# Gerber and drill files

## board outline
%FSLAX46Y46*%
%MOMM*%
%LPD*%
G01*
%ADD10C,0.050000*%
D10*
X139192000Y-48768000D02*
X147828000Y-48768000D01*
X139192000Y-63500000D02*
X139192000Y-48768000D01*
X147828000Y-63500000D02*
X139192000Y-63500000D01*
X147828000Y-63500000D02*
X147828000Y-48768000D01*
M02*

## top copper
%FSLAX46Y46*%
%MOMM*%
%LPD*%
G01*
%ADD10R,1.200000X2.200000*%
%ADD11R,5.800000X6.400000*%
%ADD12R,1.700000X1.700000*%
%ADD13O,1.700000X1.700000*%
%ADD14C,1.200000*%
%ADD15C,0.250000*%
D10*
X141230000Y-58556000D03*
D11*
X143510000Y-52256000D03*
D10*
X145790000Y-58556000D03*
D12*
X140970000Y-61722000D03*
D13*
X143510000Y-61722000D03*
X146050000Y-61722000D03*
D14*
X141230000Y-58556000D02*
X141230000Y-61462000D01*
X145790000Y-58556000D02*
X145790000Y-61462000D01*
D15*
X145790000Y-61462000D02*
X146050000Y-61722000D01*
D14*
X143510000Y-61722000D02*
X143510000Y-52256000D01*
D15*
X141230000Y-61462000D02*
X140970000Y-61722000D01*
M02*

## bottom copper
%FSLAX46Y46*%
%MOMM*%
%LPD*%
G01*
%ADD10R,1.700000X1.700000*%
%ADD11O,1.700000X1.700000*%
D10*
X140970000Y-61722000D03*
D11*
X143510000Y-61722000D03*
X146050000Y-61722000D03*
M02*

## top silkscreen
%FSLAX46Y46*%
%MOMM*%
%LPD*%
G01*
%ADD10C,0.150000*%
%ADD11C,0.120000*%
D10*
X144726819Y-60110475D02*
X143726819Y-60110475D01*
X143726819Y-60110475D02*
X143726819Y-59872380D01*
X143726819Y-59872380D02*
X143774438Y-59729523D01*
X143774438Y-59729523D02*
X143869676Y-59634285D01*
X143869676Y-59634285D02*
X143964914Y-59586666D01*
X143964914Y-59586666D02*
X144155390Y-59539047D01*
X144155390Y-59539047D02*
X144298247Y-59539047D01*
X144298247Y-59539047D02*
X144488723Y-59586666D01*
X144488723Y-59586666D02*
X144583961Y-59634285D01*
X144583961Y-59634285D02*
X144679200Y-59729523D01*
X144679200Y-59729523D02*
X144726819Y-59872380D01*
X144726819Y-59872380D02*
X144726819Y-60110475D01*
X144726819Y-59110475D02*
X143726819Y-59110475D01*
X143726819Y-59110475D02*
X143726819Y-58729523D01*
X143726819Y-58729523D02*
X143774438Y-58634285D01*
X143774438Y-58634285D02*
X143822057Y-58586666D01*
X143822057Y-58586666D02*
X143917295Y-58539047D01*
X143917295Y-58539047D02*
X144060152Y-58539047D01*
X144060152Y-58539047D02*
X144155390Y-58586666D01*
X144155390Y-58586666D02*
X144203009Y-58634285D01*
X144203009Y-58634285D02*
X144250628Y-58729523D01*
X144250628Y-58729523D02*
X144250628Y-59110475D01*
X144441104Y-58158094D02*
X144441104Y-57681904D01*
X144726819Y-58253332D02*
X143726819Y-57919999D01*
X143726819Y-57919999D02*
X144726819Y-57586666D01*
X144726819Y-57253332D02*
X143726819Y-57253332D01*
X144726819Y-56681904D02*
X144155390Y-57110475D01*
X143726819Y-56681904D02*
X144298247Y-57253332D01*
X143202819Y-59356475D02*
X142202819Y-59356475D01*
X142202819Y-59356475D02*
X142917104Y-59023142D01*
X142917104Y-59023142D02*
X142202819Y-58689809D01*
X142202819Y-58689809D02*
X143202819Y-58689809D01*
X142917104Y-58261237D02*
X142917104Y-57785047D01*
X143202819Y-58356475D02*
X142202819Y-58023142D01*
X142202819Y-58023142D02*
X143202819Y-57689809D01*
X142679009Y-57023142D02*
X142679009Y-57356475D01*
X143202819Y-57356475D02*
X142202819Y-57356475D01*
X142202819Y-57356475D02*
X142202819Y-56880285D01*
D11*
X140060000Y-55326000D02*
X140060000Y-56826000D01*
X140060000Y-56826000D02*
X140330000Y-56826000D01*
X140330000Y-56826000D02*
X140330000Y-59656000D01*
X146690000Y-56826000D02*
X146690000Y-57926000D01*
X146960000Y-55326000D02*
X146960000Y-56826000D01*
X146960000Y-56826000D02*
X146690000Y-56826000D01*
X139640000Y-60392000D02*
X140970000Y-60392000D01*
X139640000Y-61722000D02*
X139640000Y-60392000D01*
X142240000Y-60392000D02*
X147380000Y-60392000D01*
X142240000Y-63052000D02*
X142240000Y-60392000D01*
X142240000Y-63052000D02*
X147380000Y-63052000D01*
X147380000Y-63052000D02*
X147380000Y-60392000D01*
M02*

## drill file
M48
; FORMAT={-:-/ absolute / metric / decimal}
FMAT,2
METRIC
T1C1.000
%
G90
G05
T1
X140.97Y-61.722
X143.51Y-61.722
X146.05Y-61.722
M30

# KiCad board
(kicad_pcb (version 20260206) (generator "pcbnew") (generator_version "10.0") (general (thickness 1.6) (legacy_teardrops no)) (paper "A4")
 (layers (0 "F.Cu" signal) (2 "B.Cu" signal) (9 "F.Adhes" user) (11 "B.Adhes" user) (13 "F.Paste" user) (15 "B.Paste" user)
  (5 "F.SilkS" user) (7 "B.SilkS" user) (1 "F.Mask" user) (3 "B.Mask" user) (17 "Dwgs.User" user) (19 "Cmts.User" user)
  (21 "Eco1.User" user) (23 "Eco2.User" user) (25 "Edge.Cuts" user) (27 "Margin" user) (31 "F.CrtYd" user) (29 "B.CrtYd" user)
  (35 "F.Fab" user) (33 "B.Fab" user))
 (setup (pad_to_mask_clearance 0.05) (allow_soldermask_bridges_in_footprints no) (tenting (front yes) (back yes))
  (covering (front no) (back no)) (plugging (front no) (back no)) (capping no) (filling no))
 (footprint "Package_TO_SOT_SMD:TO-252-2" (layer "F.Cu") (at 143.51 54.356 90)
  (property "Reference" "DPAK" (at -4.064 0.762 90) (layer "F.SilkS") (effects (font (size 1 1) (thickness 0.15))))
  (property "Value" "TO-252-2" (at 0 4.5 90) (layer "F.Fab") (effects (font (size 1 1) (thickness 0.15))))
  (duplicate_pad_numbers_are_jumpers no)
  (fp_line (start -0.97 -3.45) (end -2.47 -3.45) (stroke (width 0.12) (type solid)) (layer "F.SilkS"))
  (fp_line (start -2.47 -3.45) (end -2.47 -3.18) (stroke (width 0.12) (type solid)) (layer "F.SilkS"))
  (fp_line (start -2.47 -3.18) (end -5.3 -3.18) (stroke (width 0.12) (type solid)) (layer "F.SilkS"))
  (fp_line (start -2.47 3.18) (end -3.57 3.18) (stroke (width 0.12) (type solid)) (layer "F.SilkS"))
  (fp_line (start -0.97 3.45) (end -2.47 3.45) (stroke (width 0.12) (type solid)) (layer "F.SilkS"))
  (fp_line (start -2.47 3.45) (end -2.47 3.18) (stroke (width 0.12) (type solid)) (layer "F.SilkS"))
  (pad "" smd rect (at 0.425 -1.525 90) (size 3.05 2.75) (layers "F.Paste"))
  (pad "" smd rect (at 0.425 1.525 90) (size 3.05 2.75) (layers "F.Paste"))
  (pad "" smd rect (at 3.775 -1.525 90) (size 3.05 2.75) (layers "F.Paste"))
  (pad "" smd rect (at 3.775 1.525 90) (size 3.05 2.75) (layers "F.Paste"))
  (pad "1" smd rect (at -4.2 -2.28 90) (size 2.2 1.2) (layers "F.Cu" "F.Mask" "F.Paste"))
  (pad "2" smd rect (at 2.1 0 90) (size 6.4 5.8) (layers "F.Cu" "F.Mask"))
  (pad "3" smd rect (at -4.2 2.28 90) (size 2.2 1.2) (layers "F.Cu" "F.Mask" "F.Paste")))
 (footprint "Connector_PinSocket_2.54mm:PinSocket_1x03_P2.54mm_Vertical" (layer "F.Cu") (at 140.97 61.722 90)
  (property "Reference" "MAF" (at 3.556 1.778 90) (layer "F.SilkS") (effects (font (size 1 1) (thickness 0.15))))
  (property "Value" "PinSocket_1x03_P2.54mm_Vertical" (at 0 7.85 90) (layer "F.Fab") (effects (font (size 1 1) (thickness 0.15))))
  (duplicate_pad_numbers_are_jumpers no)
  (fp_line (start 1.33 -1.33) (end 1.33 0) (stroke (width 0.12) (type solid)) (layer "F.SilkS"))
  (fp_line (start 0 -1.33) (end 1.33 -1.33) (stroke (width 0.12) (type solid)) (layer "F.SilkS"))
  (fp_line (start 1.33 1.27) (end 1.33 6.41) (stroke (width 0.12) (type solid)) (layer "F.SilkS"))
  (fp_line (start -1.33 1.27) (end 1.33 1.27) (stroke (width 0.12) (type solid)) (layer "F.SilkS"))
  (fp_line (start -1.33 1.27) (end -1.33 6.41) (stroke (width 0.12) (type solid)) (layer "F.SilkS"))
  (fp_line (start -1.33 6.41) (end 1.33 6.41) (stroke (width 0.12) (type solid)) (layer "F.SilkS"))
  (pad "1" thru_hole rect (at 0 0 90) (size 1.7 1.7) (drill 1) (layers "*.Cu" "*.Mask") (remove_unused_layers no))
  (pad "2" thru_hole oval (at 0 2.54 90) (size 1.7 1.7) (drill 1) (layers "*.Cu" "*.Mask") (remove_unused_layers no))
  (pad "3" thru_hole oval (at 0 5.08 90) (size 1.7 1.7) (drill 1) (layers "*.Cu" "*.Mask") (remove_unused_layers no)))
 (gr_line (start 139.192 48.768) (end 147.828 48.768) (stroke (width 0.05) (type solid)) (layer "Edge.Cuts"))
 (gr_line (start 139.192 63.5) (end 139.192 48.768) (stroke (width 0.05) (type solid)) (layer "Edge.Cuts"))
 (gr_line (start 147.828 63.5) (end 139.192 63.5) (stroke (width 0.05) (type solid)) (layer "Edge.Cuts"))
 (gr_line (start 147.828 63.5) (end 147.828 48.768) (stroke (width 0.05) (type solid)) (layer "Edge.Cuts"))
 (segment (start 141.23 58.556) (end 141.23 61.462) (width 1.2) (layer "F.Cu") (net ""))
 (segment (start 145.79 58.556) (end 145.79 61.462) (width 1.2) (layer "F.Cu") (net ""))
 (segment (start 145.79 61.462) (end 146.05 61.722) (width 0.25) (layer "F.Cu") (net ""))
 (segment (start 143.51 61.722) (end 143.51 52.256) (width 1.2) (layer "F.Cu") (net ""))
 (segment (start 141.23 61.462) (end 140.97 61.722) (width 0.25) (layer "F.Cu") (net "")))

